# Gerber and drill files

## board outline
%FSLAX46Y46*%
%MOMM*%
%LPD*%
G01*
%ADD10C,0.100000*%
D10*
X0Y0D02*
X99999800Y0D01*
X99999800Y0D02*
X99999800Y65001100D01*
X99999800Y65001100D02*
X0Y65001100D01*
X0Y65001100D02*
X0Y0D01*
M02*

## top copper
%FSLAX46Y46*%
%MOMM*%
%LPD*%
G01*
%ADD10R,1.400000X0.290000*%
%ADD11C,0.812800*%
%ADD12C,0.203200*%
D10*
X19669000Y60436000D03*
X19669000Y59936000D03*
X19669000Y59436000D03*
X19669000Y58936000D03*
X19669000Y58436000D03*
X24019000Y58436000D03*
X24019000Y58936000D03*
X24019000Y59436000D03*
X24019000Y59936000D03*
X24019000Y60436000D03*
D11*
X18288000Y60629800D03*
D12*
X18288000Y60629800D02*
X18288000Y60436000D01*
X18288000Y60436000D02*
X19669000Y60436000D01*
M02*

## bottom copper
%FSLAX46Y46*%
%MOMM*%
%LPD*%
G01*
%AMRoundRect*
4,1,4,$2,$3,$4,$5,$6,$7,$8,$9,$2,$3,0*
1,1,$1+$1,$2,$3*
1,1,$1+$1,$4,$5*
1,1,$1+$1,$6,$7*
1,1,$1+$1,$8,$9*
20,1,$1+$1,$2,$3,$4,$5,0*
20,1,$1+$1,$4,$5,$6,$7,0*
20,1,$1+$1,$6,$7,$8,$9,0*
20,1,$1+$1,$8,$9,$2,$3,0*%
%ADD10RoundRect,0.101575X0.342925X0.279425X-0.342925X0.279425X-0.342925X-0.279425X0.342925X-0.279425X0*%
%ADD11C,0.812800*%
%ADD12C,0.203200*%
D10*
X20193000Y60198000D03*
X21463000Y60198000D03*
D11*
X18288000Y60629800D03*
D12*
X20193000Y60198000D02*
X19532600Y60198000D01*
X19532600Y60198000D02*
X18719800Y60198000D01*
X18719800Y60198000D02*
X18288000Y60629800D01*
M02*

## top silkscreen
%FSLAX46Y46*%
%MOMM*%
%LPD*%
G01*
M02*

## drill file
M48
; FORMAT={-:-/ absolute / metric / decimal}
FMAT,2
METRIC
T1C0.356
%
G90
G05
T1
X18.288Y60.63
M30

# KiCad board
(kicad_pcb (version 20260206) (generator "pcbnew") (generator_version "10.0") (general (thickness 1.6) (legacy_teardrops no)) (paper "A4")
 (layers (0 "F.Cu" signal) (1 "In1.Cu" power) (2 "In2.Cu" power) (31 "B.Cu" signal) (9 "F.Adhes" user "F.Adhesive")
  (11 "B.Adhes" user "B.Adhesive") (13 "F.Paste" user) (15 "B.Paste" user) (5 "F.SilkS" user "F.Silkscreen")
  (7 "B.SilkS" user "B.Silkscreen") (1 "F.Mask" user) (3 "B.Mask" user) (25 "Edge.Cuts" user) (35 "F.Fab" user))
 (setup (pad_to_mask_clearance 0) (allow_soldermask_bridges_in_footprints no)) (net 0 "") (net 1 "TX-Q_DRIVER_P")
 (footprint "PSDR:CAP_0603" (layer "B.Cu") (at 20.8280 -60.1980 0)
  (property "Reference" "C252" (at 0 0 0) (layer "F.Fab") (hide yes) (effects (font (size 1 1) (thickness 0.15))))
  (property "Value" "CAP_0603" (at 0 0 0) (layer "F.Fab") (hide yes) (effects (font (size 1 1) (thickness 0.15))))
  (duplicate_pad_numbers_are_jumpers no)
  (pad "1" smd roundrect (at -0.6350 0.0000 -180.0000) (size 0.8890 0.7620) (layers "B.Cu" "B.Paste" "B.Mask") (roundrect_rratio 0.1333)
   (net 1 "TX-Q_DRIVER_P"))
  (pad "2" smd roundrect (at 0.6350 0.0000 -180.0000) (size 0.8890 0.7620) (layers "B.Cu" "B.Paste" "B.Mask") (roundrect_rratio 0.1333)))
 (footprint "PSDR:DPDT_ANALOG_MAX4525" (layer "F.Cu") (at 21.8440 -59.4360 0)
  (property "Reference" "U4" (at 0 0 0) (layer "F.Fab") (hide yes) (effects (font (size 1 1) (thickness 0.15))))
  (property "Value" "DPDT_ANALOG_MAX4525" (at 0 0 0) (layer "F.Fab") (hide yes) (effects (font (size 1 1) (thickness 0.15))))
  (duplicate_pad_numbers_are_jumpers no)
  (pad "1" smd rect (at -2.1750 -1.0000 0.0000) (size 1.4000 0.2900) (layers "F.Cu" "F.Paste" "F.Mask") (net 1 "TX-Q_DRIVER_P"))
  (pad "2" smd rect (at -2.1750 -0.5000 0.0000) (size 1.4000 0.2900) (layers "F.Cu" "F.Paste" "F.Mask"))
  (pad "3" smd rect (at -2.1750 0.0000 0.0000) (size 1.4000 0.2900) (layers "F.Cu" "F.Paste" "F.Mask"))
  (pad "4" smd rect (at -2.1750 0.5000 0.0000) (size 1.4000 0.2900) (layers "F.Cu" "F.Paste" "F.Mask"))
  (pad "5" smd rect (at -2.1750 1.0000 0.0000) (size 1.4000 0.2900) (layers "F.Cu" "F.Paste" "F.Mask"))
  (pad "6" smd rect (at 2.1750 1.0000 0.0000) (size 1.4000 0.2900) (layers "F.Cu" "F.Paste" "F.Mask"))
  (pad "7" smd rect (at 2.1750 0.5000 0.0000) (size 1.4000 0.2900) (layers "F.Cu" "F.Paste" "F.Mask"))
  (pad "8" smd rect (at 2.1750 0.0000 0.0000) (size 1.4000 0.2900) (layers "F.Cu" "F.Paste" "F.Mask"))
  (pad "9" smd rect (at 2.1750 -0.5000 0.0000) (size 1.4000 0.2900) (layers "F.Cu" "F.Paste" "F.Mask"))
  (pad "10" smd rect (at 2.1750 -1.0000 0.0000) (size 1.4000 0.2900) (layers "F.Cu" "F.Paste" "F.Mask")))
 (segment (start 20.1930 -60.1980) (end 19.5326 -60.1980) (width 0.2032) (layer "B.Cu") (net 1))
 (segment (start 19.5326 -60.1980) (end 18.7198 -60.1980) (width 0.2032) (layer "B.Cu") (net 1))
 (segment (start 18.7198 -60.1980) (end 18.2880 -60.6298) (width 0.2032) (layer "B.Cu") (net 1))
 (segment (start 18.2880 -60.6298) (end 18.2880 -60.4360) (width 0.2032) (layer "F.Cu") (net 1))
 (segment (start 18.2880 -60.4360) (end 19.6690 -60.4360) (width 0.2032) (layer "F.Cu") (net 1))
 (via (at 18.2880 -60.6298) (size 0.8128) (drill 0.3556) (layers "F.Cu" "B.Cu") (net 1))
 (gr_line (start 0.0000 0.0000) (end 99.9998 0.0000) (stroke (width 0.1) (type default)) (layer "Edge.Cuts"))
 (gr_line (start 99.9998 0.0000) (end 99.9998 -65.0011) (stroke (width 0.1) (type default)) (layer "Edge.Cuts"))
 (gr_line (start 99.9998 -65.0011) (end 0.0000 -65.0011) (stroke (width 0.1) (type default)) (layer "Edge.Cuts"))
 (gr_line (start 0.0000 -65.0011) (end 0.0000 0.0000) (stroke (width 0.1) (type default)) (layer "Edge.Cuts")))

